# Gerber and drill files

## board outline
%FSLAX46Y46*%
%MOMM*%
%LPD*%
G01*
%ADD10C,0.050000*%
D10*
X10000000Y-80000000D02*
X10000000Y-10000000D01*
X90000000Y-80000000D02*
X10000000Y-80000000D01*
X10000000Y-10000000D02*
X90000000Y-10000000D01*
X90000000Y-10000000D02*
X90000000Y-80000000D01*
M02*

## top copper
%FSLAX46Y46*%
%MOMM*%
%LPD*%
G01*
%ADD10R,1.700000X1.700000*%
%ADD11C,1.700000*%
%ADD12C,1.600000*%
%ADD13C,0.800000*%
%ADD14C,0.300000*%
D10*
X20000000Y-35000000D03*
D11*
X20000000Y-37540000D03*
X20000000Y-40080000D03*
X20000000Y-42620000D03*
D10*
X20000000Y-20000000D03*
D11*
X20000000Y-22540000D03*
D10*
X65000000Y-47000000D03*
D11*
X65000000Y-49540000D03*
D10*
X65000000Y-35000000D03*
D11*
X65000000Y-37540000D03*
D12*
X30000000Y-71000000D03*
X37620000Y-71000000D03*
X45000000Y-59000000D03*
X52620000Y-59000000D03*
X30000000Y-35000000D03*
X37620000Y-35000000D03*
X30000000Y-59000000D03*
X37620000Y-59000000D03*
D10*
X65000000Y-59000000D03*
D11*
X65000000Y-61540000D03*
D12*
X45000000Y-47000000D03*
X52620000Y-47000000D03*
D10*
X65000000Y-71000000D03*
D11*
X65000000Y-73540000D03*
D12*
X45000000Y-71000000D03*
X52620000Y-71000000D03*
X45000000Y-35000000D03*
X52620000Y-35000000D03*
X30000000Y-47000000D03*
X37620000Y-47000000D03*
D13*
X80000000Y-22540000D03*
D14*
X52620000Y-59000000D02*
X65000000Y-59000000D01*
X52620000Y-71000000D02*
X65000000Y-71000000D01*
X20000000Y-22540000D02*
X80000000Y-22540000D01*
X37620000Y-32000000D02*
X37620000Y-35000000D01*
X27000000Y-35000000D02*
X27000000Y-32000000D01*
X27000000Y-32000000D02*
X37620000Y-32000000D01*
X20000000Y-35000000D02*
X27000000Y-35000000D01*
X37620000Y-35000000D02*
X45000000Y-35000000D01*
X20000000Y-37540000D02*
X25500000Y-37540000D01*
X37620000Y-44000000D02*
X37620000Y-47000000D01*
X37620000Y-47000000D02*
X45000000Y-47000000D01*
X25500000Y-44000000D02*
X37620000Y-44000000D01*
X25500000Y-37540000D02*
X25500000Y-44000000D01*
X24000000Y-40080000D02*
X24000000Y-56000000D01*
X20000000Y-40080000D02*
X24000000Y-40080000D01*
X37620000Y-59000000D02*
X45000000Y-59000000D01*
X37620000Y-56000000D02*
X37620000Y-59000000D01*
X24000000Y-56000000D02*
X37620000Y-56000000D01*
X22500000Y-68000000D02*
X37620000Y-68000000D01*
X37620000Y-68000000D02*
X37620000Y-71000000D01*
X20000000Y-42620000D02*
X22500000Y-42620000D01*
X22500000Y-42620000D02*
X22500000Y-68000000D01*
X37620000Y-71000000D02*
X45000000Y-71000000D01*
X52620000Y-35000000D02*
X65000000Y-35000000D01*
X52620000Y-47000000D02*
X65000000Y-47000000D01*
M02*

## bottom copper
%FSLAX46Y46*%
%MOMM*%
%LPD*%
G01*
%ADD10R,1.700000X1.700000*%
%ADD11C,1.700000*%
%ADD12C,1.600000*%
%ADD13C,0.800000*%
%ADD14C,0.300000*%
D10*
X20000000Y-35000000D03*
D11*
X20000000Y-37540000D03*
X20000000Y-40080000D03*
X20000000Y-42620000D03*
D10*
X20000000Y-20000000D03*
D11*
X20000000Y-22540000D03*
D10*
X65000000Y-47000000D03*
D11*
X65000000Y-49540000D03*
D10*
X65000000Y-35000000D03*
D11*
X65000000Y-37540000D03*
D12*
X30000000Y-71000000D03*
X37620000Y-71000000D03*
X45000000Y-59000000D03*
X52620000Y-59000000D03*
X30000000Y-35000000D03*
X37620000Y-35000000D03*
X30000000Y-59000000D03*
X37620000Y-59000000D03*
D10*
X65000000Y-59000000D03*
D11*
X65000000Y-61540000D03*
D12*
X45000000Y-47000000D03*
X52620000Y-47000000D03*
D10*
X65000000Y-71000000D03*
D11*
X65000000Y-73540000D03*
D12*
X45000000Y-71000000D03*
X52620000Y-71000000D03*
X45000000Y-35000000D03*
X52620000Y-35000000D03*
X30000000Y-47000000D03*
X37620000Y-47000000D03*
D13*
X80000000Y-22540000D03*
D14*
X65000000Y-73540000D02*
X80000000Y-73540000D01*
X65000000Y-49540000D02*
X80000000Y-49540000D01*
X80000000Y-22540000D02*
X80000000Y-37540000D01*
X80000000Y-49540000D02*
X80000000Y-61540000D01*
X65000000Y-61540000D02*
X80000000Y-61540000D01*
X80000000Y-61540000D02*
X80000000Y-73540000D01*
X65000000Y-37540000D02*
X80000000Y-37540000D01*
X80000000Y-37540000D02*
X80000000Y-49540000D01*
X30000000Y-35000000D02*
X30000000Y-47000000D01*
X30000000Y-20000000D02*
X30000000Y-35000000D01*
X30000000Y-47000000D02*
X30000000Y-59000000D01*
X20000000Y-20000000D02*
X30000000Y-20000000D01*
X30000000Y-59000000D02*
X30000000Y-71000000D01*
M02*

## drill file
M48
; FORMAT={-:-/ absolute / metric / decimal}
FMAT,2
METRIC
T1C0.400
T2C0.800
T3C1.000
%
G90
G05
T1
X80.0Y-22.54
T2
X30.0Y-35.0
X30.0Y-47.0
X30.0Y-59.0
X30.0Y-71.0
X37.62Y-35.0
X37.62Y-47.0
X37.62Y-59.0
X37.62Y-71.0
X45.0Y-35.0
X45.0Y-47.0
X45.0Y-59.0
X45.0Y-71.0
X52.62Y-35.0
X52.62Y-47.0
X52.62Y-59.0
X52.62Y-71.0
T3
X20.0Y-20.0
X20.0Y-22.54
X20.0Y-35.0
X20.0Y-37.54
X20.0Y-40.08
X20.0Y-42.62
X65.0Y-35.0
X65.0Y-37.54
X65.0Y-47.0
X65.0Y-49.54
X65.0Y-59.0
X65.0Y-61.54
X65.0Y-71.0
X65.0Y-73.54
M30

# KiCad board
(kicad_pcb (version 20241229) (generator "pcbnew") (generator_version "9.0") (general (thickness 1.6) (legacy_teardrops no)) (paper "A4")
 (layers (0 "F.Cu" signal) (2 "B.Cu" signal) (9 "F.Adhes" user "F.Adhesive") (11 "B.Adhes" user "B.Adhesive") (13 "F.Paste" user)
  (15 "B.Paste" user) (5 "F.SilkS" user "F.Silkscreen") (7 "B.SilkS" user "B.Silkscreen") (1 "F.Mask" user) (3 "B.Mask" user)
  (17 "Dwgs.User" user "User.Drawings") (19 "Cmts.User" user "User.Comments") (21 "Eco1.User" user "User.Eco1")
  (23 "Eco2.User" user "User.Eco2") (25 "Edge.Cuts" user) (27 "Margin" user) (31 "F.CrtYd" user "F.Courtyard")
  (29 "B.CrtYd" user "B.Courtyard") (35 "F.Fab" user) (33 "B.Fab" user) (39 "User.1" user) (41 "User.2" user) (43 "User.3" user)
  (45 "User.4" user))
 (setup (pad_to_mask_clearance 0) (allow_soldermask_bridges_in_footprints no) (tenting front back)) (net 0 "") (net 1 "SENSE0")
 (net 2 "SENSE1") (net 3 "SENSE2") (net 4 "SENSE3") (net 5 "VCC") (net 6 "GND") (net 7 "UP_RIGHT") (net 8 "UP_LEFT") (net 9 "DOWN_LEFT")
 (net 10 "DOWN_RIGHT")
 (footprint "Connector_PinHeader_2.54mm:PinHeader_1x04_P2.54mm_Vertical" (layer "F.Cu") (at 20 35)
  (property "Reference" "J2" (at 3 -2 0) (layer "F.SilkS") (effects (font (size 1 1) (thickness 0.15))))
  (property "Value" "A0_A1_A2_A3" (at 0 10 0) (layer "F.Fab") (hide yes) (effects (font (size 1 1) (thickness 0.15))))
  (pad "1" thru_hole rect (at 0 0) (size 1.7 1.7) (drill 1) (layers "*.Cu" "*.Mask") (remove_unused_layers no) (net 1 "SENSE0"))
  (pad "2" thru_hole circle (at 0 2.54) (size 1.7 1.7) (drill 1) (layers "*.Cu" "*.Mask") (remove_unused_layers no) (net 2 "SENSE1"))
  (pad "3" thru_hole circle (at 0 5.08) (size 1.7 1.7) (drill 1) (layers "*.Cu" "*.Mask") (remove_unused_layers no) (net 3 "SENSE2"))
  (pad "4" thru_hole circle (at 0 7.62) (size 1.7 1.7) (drill 1) (layers "*.Cu" "*.Mask") (remove_unused_layers no) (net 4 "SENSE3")))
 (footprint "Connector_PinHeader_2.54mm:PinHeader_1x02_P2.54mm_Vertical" (layer "F.Cu") (at 20 20)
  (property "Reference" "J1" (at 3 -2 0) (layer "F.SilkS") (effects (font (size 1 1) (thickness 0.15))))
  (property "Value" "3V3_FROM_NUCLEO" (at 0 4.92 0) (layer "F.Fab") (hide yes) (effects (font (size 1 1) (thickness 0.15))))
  (pad "1" thru_hole rect (at 0 0) (size 1.7 1.7) (drill 1) (layers "*.Cu" "*.Mask") (remove_unused_layers no) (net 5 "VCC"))
  (pad "2" thru_hole circle (at 0 2.54) (size 1.7 1.7) (drill 1) (layers "*.Cu" "*.Mask") (remove_unused_layers no) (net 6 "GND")))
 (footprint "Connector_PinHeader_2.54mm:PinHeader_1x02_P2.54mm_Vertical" (layer "F.Cu") (at 65 47)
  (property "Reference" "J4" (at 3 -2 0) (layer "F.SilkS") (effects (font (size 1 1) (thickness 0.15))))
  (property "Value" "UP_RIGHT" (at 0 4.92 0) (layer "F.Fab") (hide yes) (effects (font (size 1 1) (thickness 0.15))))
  (pad "1" thru_hole rect (at 0 0) (size 1.7 1.7) (drill 1) (layers "*.Cu" "*.Mask") (remove_unused_layers no) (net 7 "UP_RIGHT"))
  (pad "2" thru_hole circle (at 0 2.54) (size 1.7 1.7) (drill 1) (layers "*.Cu" "*.Mask") (remove_unused_layers no) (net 6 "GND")))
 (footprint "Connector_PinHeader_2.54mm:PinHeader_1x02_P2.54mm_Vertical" (layer "F.Cu") (at 65 35)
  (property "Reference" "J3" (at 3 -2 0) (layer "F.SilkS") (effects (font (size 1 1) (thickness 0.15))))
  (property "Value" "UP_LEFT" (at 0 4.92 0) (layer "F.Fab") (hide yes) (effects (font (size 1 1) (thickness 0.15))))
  (pad "1" thru_hole rect (at 0 0) (size 1.7 1.7) (drill 1) (layers "*.Cu" "*.Mask") (remove_unused_layers no) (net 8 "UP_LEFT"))
  (pad "2" thru_hole circle (at 0 2.54) (size 1.7 1.7) (drill 1) (layers "*.Cu" "*.Mask") (remove_unused_layers no) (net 6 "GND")))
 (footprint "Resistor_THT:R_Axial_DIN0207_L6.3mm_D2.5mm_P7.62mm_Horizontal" (layer "F.Cu") (at 30 71)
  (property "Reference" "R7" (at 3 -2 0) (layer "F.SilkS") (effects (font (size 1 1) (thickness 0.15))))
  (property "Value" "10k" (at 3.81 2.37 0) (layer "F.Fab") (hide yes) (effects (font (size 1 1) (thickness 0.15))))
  (pad "1" thru_hole circle (at 0 0) (size 1.6 1.6) (drill 0.8) (layers "*.Cu" "*.Mask") (remove_unused_layers no) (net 5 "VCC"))
  (pad "2" thru_hole circle (at 7.62 0) (size 1.6 1.6) (drill 0.8) (layers "*.Cu" "*.Mask") (remove_unused_layers no) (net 4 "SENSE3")))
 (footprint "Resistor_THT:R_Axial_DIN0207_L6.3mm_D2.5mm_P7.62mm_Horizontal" (layer "F.Cu") (at 45 59)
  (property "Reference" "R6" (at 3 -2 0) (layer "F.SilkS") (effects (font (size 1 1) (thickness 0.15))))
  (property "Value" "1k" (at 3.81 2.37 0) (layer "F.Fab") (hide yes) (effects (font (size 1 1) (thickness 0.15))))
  (pad "1" thru_hole circle (at 0 0) (size 1.6 1.6) (drill 0.8) (layers "*.Cu" "*.Mask") (remove_unused_layers no) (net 3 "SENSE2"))
  (pad "2" thru_hole circle (at 7.62 0) (size 1.6 1.6) (drill 0.8) (layers "*.Cu" "*.Mask") (remove_unused_layers no) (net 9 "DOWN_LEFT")))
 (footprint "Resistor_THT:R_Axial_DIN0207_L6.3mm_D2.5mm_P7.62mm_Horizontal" (layer "F.Cu") (at 30 35)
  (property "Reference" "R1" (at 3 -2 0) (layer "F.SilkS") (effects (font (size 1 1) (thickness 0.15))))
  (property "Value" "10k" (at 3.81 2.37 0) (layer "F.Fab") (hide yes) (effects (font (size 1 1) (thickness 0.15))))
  (pad "1" thru_hole circle (at 0 0) (size 1.6 1.6) (drill 0.8) (layers "*.Cu" "*.Mask") (remove_unused_layers no) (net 5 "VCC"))
  (pad "2" thru_hole circle (at 7.62 0) (size 1.6 1.6) (drill 0.8) (layers "*.Cu" "*.Mask") (remove_unused_layers no) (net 1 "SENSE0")))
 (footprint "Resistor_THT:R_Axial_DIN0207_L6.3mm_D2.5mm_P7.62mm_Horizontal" (layer "F.Cu") (at 30 59)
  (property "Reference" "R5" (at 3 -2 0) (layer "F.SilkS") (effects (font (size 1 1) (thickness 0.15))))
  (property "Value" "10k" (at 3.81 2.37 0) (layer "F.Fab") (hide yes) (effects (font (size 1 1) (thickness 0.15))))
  (pad "1" thru_hole circle (at 0 0) (size 1.6 1.6) (drill 0.8) (layers "*.Cu" "*.Mask") (remove_unused_layers no) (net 5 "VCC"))
  (pad "2" thru_hole circle (at 7.62 0) (size 1.6 1.6) (drill 0.8) (layers "*.Cu" "*.Mask") (remove_unused_layers no) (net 3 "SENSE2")))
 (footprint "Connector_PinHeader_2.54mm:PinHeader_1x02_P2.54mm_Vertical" (layer "F.Cu") (at 65 59)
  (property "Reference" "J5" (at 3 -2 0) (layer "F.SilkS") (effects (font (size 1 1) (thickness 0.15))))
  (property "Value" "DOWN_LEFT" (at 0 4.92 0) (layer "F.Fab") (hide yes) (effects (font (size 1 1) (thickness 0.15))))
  (pad "1" thru_hole rect (at 0 0) (size 1.7 1.7) (drill 1) (layers "*.Cu" "*.Mask") (remove_unused_layers no) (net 9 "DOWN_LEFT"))
  (pad "2" thru_hole circle (at 0 2.54) (size 1.7 1.7) (drill 1) (layers "*.Cu" "*.Mask") (remove_unused_layers no) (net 6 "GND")))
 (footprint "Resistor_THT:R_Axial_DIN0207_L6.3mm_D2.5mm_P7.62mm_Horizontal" (layer "F.Cu") (at 45 47)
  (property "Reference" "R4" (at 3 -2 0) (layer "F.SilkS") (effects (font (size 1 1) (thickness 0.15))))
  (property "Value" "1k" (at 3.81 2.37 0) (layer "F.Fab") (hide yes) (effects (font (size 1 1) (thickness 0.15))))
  (pad "1" thru_hole circle (at 0 0) (size 1.6 1.6) (drill 0.8) (layers "*.Cu" "*.Mask") (remove_unused_layers no) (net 2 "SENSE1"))
  (pad "2" thru_hole circle (at 7.62 0) (size 1.6 1.6) (drill 0.8) (layers "*.Cu" "*.Mask") (remove_unused_layers no) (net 7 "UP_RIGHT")))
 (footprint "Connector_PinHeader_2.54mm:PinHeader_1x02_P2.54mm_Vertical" (layer "F.Cu") (at 65 71)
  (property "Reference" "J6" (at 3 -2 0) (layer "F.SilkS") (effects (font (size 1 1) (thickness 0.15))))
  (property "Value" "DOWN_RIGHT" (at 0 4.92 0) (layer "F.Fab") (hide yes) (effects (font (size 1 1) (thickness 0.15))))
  (pad "1" thru_hole rect (at 0 0) (size 1.7 1.7) (drill 1) (layers "*.Cu" "*.Mask") (remove_unused_layers no) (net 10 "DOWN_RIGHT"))
  (pad "2" thru_hole circle (at 0 2.54) (size 1.7 1.7) (drill 1) (layers "*.Cu" "*.Mask") (remove_unused_layers no) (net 6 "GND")))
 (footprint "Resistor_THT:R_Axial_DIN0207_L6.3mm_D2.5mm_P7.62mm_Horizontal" (layer "F.Cu") (at 45 71)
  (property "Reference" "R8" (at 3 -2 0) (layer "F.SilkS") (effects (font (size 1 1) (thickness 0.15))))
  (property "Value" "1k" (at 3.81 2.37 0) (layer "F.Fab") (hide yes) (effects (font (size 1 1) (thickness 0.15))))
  (pad "1" thru_hole circle (at 0 0) (size 1.6 1.6) (drill 0.8) (layers "*.Cu" "*.Mask") (remove_unused_layers no) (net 4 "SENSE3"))
  (pad "2" thru_hole circle (at 7.62 0) (size 1.6 1.6) (drill 0.8) (layers "*.Cu" "*.Mask") (remove_unused_layers no) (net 10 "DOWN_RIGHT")))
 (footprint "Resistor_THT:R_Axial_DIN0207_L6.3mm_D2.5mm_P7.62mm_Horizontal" (layer "F.Cu") (at 45 35)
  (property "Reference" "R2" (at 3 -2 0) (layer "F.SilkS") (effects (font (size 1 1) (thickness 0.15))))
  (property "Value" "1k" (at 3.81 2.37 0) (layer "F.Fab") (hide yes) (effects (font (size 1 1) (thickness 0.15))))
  (pad "1" thru_hole circle (at 0 0) (size 1.6 1.6) (drill 0.8) (layers "*.Cu" "*.Mask") (remove_unused_layers no) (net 1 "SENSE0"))
  (pad "2" thru_hole circle (at 7.62 0) (size 1.6 1.6) (drill 0.8) (layers "*.Cu" "*.Mask") (remove_unused_layers no) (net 8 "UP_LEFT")))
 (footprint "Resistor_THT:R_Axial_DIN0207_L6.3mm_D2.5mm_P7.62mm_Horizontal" (layer "F.Cu") (at 30 47)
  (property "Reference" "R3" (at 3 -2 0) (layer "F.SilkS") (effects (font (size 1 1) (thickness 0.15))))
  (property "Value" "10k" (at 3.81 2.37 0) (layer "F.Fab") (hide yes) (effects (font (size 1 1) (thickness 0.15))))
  (pad "1" thru_hole circle (at 0 0) (size 1.6 1.6) (drill 0.8) (layers "*.Cu" "*.Mask") (remove_unused_layers no) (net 5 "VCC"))
  (pad "2" thru_hole circle (at 7.62 0) (size 1.6 1.6) (drill 0.8) (layers "*.Cu" "*.Mask") (remove_unused_layers no) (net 2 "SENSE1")))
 (gr_line (start 10 80) (end 10 10) (stroke (width 0.05) (type default)) (layer "Edge.Cuts"))
 (gr_line (start 90 80) (end 10 80) (stroke (width 0.05) (type default)) (layer "Edge.Cuts"))
 (gr_line (start 10 10) (end 90 10) (stroke (width 0.05) (type default)) (layer "Edge.Cuts"))
 (gr_line (start 90 10) (end 90 80) (stroke (width 0.05) (type default)) (layer "Edge.Cuts"))
 (segment (start 52.62 59) (end 65 59) (width 0.3) (layer "F.Cu") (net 9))
 (segment (start 52.62 71) (end 65 71) (width 0.3) (layer "F.Cu") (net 10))
 (segment (start 20 22.54) (end 80 22.54) (width 0.3) (layer "F.Cu") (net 6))
 (via (at 80 22.54) (size 0.8) (drill 0.4) (layers "F.Cu" "B.Cu") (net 6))
 (segment (start 65 73.54) (end 80 73.54) (width 0.3) (layer "B.Cu") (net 6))
 (segment (start 65 49.54) (end 80 49.54) (width 0.3) (layer "B.Cu") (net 6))
 (segment (start 80 22.54) (end 80 37.54) (width 0.3) (layer "B.Cu") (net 6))
 (segment (start 80 49.54) (end 80 61.54) (width 0.3) (layer "B.Cu") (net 6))
 (segment (start 65 61.54) (end 80 61.54) (width 0.3) (layer "B.Cu") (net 6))
 (segment (start 80 61.54) (end 80 73.54) (width 0.3) (layer "B.Cu") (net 6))
 (segment (start 65 37.54) (end 80 37.54) (width 0.3) (layer "B.Cu") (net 6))
 (segment (start 80 37.54) (end 80 49.54) (width 0.3) (layer "B.Cu") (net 6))
 (segment (start 37.62 32) (end 37.62 35) (width 0.3) (layer "F.Cu") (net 1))
 (segment (start 27 35) (end 27 32) (width 0.3) (layer "F.Cu") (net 1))
 (segment (start 27 32) (end 37.62 32) (width 0.3) (layer "F.Cu") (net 1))
 (segment (start 20 35) (end 27 35) (width 0.3) (layer "F.Cu") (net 1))
 (segment (start 37.62 35) (end 45 35) (width 0.3) (layer "F.Cu") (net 1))
 (segment (start 20 37.54) (end 25.5 37.54) (width 0.3) (layer "F.Cu") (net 2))
 (segment (start 37.62 44) (end 37.62 47) (width 0.3) (layer "F.Cu") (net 2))
 (segment (start 37.62 47) (end 45 47) (width 0.3) (layer "F.Cu") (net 2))
 (segment (start 25.5 44) (end 37.62 44) (width 0.3) (layer "F.Cu") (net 2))
 (segment (start 25.5 37.54) (end 25.5 44) (width 0.3) (layer "F.Cu") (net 2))
 (segment (start 24 40.08) (end 24 56) (width 0.3) (layer "F.Cu") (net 3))
 (segment (start 20 40.08) (end 24 40.08) (width 0.3) (layer "F.Cu") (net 3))
 (segment (start 37.62 59) (end 45 59) (width 0.3) (layer "F.Cu") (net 3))
 (segment (start 37.62 56) (end 37.62 59) (width 0.3) (layer "F.Cu") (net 3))
 (segment (start 24 56) (end 37.62 56) (width 0.3) (layer "F.Cu") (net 3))
 (segment (start 22.5 68) (end 37.62 68) (width 0.3) (layer "F.Cu") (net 4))
 (segment (start 37.62 68) (end 37.62 71) (width 0.3) (layer "F.Cu") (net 4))
 (segment (start 20 42.62) (end 22.5 42.62) (width 0.3) (layer "F.Cu") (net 4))
 (segment (start 22.5 42.62) (end 22.5 68) (width 0.3) (layer "F.Cu") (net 4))
 (segment (start 37.62 71) (end 45 71) (width 0.3) (layer "F.Cu") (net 4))
 (segment (start 52.62 35) (end 65 35) (width 0.3) (layer "F.Cu") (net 8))
 (segment (start 52.62 47) (end 65 47) (width 0.3) (layer "F.Cu") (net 7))
 (segment (start 30 35) (end 30 47) (width 0.3) (layer "B.Cu") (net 5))
 (segment (start 30 20) (end 30 35) (width 0.3) (layer "B.Cu") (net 5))
 (segment (start 30 47) (end 30 59) (width 0.3) (layer "B.Cu") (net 5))
 (segment (start 20 20) (end 30 20) (width 0.3) (layer "B.Cu") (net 5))
 (segment (start 30 59) (end 30 71) (width 0.3) (layer "B.Cu") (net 5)))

